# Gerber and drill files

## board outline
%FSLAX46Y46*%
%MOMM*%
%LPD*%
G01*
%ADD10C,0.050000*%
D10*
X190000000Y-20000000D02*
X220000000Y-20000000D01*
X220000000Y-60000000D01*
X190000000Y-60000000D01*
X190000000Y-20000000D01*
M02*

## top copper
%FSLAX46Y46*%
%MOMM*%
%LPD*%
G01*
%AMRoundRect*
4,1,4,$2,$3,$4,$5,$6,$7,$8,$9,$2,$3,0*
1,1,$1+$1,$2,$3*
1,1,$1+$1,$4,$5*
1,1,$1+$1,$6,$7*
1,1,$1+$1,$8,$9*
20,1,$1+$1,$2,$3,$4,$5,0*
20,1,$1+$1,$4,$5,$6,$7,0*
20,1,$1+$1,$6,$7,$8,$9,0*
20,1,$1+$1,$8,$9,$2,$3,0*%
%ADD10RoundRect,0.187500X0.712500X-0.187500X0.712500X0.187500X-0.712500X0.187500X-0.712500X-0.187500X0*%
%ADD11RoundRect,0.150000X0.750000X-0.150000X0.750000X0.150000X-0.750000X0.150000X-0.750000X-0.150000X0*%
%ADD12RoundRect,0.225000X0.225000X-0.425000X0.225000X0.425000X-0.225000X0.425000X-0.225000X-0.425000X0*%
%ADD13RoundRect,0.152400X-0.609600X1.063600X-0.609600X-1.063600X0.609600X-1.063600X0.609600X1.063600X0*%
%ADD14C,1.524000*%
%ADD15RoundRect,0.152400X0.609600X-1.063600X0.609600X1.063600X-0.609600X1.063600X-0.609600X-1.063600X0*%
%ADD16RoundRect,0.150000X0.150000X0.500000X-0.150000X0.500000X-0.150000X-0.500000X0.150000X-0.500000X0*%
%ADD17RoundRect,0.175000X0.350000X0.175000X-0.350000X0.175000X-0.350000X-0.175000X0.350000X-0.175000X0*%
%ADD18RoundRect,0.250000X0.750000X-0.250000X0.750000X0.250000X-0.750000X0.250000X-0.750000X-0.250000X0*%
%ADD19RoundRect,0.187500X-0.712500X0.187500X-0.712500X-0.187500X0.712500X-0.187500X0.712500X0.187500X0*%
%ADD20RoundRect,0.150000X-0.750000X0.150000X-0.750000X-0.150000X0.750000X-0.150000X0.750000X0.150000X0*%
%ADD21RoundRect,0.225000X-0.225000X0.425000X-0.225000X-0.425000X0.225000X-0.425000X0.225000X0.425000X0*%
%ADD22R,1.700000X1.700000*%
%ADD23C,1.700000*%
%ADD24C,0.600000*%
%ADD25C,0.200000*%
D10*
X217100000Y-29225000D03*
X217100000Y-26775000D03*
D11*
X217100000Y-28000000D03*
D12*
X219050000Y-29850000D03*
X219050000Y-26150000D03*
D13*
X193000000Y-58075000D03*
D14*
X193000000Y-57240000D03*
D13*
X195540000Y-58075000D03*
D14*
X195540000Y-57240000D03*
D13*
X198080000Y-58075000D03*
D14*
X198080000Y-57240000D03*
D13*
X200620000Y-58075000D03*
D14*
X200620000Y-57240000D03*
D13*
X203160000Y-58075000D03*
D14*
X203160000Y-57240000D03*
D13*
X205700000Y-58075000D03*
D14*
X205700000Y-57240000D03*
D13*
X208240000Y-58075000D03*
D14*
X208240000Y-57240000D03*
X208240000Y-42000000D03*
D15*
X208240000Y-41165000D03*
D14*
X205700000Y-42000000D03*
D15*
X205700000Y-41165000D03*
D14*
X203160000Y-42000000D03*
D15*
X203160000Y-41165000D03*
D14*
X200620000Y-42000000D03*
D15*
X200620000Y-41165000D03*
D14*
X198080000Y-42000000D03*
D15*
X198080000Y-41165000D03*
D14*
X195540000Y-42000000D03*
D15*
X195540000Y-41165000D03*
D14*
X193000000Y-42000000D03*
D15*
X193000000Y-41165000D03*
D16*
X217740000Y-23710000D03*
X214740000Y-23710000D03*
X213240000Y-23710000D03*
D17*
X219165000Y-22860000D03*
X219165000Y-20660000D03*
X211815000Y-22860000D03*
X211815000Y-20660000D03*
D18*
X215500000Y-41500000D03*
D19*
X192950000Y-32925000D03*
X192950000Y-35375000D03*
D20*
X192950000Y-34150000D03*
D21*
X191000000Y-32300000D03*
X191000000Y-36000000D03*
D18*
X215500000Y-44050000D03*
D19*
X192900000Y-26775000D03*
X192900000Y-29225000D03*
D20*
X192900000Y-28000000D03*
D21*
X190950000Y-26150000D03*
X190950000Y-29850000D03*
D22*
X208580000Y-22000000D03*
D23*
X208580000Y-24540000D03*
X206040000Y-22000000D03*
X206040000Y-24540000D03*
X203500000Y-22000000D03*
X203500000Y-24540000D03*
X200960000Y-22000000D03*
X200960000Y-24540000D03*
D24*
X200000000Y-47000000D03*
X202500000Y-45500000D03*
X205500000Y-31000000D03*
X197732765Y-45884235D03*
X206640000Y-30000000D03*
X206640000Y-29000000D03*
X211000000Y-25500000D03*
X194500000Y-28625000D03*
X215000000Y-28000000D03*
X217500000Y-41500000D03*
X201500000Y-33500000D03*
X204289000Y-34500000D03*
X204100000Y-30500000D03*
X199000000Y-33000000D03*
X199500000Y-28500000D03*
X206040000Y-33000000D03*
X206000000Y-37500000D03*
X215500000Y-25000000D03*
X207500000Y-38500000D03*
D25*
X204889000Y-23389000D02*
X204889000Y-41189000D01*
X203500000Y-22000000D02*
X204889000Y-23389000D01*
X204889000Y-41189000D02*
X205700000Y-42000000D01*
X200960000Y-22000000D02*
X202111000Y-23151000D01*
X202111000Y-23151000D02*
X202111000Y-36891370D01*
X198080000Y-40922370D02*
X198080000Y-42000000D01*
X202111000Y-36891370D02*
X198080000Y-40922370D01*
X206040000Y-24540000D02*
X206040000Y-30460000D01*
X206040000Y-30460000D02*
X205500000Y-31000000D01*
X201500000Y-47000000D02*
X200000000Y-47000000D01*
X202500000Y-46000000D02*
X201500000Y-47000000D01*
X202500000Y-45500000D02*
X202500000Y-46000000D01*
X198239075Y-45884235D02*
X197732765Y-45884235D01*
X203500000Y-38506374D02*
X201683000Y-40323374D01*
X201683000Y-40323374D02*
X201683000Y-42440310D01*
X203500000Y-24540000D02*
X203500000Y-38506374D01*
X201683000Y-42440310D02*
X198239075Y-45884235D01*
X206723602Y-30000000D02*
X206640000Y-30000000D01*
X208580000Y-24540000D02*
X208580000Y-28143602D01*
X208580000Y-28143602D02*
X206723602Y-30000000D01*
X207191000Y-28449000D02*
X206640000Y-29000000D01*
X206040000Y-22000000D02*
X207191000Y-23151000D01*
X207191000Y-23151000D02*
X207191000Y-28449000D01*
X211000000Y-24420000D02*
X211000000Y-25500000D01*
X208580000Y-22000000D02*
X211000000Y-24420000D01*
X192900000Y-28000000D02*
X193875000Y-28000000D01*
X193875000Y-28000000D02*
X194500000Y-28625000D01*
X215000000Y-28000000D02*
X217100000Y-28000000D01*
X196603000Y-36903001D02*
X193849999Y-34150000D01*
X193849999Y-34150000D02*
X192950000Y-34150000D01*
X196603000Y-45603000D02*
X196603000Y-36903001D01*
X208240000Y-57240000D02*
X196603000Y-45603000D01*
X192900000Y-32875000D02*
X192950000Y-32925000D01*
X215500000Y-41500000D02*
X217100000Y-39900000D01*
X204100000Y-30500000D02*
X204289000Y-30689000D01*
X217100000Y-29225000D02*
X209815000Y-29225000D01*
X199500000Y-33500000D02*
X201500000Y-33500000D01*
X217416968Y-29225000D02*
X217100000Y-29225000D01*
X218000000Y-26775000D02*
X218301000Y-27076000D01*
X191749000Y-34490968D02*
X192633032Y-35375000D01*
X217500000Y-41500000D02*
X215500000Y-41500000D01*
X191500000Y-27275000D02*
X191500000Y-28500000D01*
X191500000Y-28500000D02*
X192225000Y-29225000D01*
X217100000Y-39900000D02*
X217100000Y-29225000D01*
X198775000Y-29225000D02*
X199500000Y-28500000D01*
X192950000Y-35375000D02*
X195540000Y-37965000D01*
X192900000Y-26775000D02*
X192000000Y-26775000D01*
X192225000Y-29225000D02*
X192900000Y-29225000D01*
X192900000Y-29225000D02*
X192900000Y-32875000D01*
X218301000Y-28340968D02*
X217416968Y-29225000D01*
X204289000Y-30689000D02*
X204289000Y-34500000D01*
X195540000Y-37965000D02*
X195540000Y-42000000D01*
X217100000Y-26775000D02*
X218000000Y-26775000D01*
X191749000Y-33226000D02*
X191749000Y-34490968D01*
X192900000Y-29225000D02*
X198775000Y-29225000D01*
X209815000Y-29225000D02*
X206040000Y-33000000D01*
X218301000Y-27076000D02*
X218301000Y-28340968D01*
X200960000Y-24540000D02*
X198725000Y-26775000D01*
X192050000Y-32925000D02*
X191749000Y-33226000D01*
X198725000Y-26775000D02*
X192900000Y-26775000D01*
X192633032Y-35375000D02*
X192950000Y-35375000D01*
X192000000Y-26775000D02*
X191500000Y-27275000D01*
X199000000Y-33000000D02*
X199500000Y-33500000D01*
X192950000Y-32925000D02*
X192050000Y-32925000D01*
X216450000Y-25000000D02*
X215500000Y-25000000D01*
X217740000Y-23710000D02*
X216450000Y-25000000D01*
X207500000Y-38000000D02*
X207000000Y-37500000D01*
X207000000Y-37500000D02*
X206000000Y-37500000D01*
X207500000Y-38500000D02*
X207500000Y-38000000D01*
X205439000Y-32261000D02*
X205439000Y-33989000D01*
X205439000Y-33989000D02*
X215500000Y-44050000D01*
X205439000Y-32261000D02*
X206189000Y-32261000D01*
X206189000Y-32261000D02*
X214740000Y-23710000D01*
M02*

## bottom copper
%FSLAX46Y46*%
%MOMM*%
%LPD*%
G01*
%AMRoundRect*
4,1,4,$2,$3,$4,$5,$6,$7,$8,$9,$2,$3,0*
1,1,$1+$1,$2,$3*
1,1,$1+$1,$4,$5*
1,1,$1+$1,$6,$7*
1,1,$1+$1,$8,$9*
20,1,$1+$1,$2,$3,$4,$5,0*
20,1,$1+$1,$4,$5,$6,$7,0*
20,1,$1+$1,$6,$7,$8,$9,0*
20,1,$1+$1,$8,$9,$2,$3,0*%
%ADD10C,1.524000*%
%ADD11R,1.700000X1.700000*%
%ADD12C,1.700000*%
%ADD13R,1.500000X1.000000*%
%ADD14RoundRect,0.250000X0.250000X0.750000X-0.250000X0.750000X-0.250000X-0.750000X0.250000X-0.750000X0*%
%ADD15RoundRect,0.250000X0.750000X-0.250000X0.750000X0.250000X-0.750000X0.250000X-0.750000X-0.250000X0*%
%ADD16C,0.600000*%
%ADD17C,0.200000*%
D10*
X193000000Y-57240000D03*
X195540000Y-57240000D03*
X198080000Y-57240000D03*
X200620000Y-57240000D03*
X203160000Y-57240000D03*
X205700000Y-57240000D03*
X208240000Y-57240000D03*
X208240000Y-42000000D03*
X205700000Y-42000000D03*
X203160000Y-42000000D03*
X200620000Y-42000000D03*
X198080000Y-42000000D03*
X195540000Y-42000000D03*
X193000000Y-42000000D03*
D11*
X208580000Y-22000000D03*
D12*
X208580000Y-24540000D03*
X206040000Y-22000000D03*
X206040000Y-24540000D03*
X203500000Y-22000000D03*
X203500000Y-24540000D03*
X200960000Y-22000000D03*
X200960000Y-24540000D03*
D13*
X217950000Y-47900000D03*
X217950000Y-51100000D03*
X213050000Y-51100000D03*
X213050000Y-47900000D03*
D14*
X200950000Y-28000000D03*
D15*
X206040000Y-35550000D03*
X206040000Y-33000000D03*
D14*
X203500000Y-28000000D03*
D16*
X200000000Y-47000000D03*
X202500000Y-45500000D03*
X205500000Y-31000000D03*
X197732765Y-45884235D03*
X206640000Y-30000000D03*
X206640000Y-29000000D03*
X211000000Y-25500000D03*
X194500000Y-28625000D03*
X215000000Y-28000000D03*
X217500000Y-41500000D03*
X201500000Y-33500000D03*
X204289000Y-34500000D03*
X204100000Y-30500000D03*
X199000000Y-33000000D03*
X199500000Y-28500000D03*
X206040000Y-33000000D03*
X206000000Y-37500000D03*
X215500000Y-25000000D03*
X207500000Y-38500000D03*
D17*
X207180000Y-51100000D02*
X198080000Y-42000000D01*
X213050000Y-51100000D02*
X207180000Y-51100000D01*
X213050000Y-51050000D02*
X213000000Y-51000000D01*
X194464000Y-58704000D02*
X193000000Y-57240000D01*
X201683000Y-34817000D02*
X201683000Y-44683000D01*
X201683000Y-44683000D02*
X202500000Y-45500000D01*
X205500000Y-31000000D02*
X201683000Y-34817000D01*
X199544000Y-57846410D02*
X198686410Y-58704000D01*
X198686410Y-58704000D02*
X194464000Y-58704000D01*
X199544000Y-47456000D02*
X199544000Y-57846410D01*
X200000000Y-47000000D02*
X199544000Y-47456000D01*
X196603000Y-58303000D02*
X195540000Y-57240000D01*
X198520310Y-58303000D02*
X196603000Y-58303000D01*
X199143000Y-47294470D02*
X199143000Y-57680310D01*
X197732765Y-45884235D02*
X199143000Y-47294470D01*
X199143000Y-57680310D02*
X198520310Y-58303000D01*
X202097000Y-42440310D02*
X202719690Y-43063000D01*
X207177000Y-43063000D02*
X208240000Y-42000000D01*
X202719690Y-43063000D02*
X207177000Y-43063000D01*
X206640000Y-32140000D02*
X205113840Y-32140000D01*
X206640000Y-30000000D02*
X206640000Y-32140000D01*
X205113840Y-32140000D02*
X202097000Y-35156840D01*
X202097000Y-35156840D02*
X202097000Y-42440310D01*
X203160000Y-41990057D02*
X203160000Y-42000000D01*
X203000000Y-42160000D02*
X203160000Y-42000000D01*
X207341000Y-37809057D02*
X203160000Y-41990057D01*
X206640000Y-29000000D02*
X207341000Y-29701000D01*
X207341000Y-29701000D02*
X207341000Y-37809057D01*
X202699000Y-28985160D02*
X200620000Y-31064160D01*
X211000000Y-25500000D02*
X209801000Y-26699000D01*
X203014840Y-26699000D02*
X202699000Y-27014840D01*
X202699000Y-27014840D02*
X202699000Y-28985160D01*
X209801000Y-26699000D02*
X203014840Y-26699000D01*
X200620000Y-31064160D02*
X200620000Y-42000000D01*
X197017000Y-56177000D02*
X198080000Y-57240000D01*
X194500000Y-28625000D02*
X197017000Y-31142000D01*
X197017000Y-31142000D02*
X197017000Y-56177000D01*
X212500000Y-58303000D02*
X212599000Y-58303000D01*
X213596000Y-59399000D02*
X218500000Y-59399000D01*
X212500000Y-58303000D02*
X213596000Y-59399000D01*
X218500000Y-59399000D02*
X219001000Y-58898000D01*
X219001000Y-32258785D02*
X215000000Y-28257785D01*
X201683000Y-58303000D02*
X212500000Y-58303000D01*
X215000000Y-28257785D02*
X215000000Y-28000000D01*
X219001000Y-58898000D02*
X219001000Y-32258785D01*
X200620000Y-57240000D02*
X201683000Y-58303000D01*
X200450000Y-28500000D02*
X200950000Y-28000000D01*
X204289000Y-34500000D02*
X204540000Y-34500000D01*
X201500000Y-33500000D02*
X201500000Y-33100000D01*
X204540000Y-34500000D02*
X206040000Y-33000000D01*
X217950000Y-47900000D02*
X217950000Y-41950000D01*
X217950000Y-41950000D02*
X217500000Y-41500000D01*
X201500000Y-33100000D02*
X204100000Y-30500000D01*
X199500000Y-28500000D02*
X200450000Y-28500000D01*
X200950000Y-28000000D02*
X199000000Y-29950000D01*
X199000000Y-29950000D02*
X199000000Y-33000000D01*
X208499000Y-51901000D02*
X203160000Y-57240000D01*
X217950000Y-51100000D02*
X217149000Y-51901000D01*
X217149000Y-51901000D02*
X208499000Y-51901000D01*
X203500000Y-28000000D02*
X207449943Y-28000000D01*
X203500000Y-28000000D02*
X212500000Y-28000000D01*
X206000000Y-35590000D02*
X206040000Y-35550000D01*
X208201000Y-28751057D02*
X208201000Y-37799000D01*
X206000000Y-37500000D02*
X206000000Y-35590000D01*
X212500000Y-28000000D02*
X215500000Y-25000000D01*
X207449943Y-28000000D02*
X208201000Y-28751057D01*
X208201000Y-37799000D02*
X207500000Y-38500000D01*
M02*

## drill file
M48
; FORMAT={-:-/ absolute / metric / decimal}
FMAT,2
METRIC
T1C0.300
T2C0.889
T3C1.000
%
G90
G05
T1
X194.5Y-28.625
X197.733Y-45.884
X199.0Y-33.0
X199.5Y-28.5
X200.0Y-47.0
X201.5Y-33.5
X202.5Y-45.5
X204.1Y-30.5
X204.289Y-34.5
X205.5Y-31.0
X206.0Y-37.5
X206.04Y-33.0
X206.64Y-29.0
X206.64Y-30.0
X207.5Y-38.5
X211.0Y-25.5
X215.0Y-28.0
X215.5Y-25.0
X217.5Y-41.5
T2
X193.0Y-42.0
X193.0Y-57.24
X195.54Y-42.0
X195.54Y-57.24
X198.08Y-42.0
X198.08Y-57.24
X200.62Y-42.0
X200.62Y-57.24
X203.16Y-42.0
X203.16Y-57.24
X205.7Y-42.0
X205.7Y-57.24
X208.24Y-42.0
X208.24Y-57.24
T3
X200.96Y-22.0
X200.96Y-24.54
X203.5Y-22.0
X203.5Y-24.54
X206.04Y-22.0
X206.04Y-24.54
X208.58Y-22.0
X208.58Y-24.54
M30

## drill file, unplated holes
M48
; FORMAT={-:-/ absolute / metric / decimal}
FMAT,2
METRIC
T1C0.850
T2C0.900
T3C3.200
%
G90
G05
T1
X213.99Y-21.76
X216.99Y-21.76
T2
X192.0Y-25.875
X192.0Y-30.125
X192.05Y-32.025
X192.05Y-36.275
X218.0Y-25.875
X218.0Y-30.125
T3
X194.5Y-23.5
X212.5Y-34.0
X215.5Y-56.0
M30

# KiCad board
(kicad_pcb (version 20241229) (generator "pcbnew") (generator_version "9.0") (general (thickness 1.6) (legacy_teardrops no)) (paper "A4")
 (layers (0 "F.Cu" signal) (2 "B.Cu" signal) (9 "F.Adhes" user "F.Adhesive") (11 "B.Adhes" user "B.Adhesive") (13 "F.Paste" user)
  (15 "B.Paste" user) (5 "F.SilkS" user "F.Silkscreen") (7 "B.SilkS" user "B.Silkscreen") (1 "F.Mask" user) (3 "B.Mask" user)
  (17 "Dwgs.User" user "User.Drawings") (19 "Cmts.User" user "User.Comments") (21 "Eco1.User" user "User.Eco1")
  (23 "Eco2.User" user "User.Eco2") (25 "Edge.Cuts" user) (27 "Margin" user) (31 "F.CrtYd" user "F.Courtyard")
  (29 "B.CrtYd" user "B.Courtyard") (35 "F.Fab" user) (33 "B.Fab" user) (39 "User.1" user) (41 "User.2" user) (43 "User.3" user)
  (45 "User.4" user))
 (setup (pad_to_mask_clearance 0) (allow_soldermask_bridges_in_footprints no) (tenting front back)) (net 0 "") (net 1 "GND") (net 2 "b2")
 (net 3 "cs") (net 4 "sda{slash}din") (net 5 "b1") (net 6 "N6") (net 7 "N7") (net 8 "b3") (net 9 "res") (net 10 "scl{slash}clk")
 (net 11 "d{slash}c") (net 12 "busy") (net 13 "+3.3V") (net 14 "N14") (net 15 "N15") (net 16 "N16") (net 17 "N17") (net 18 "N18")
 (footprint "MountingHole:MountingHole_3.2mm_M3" (layer "F.Cu") (at 215.5 56)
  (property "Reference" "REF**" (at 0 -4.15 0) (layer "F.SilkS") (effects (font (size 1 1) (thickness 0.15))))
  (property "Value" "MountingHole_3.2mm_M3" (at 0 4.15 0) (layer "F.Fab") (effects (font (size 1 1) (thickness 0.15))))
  (pad "" np_thru_hole circle (at 0 0) (size 3.2 3.2) (drill 3.2) (layers "*.Cu" "*.Mask")))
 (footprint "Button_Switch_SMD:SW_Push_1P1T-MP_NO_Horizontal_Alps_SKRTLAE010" (layer "F.Cu") (at 218 28 90)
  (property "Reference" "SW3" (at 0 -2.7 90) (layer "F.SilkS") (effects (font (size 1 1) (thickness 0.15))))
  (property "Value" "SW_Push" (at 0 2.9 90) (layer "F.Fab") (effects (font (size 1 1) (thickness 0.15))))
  (pad "" np_thru_hole circle (at -2.125 0 90) (size 0.9 0.9) (drill 0.9) (layers "*.Cu" "*.Mask"))
  (pad "" np_thru_hole circle (at 2.125 0 90) (size 0.9 0.9) (drill 0.9) (layers "*.Cu" "*.Mask"))
  (pad "1" smd roundrect (at -1.225 -0.9 90) (size 0.75 1.8) (layers "F.Cu" "F.Mask" "F.Paste") (roundrect_rratio 0.25) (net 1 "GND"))
  (pad "1" smd roundrect (at 1.225 -0.9 90) (size 0.75 1.8) (layers "F.Cu" "F.Mask" "F.Paste") (roundrect_rratio 0.25) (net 1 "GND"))
  (pad "2" smd roundrect (at 0 -0.9 90) (size 0.6 1.8) (layers "F.Cu" "F.Mask" "F.Paste") (roundrect_rratio 0.25) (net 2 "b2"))
  (pad "MP" smd roundrect (at -1.85 1.05 90) (size 1.3 0.9) (layers "F.Cu" "F.Mask" "F.Paste") (roundrect_rratio 0.25))
  (pad "MP" smd roundrect (at 1.85 1.05 90) (size 1.3 0.9) (layers "F.Cu" "F.Mask" "F.Paste") (roundrect_rratio 0.25)))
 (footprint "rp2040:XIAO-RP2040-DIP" (layer "F.Cu") (at 200.62 49.62 90)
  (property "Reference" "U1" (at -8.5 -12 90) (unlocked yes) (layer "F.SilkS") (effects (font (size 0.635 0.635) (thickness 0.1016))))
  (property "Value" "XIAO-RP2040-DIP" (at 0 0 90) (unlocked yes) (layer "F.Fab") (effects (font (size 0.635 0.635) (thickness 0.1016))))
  (pad "1" smd roundrect (at -8.455 -7.62 270) (size 2.432 1.524) (layers "F.Cu" "F.Mask") (roundrect_rratio 0.1) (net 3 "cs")
   (thermal_bridge_angle 45))
  (pad "1" thru_hole circle (at -7.62 -7.62 270) (size 1.524 1.524) (drill 0.889) (layers "*.Cu" "*.Mask") (remove_unused_layers no)
   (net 3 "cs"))
  (pad "2" smd roundrect (at -8.455 -5.08 270) (size 2.432 1.524) (layers "F.Cu" "F.Mask") (roundrect_rratio 0.1) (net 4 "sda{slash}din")
   (thermal_bridge_angle 45))
  (pad "2" thru_hole circle (at -7.62 -5.08 270) (size 1.524 1.524) (drill 0.889) (layers "*.Cu" "*.Mask") (remove_unused_layers no)
   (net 4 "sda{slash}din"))
  (pad "3" smd roundrect (at -8.455 -2.54 270) (size 2.432 1.524) (layers "F.Cu" "F.Mask") (roundrect_rratio 0.1) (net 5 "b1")
   (thermal_bridge_angle 45))
  (pad "3" thru_hole circle (at -7.62 -2.54 270) (size 1.524 1.524) (drill 0.889) (layers "*.Cu" "*.Mask") (remove_unused_layers no)
   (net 5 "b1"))
  (pad "4" smd roundrect (at -8.455 0 270) (size 2.432 1.524) (layers "F.Cu" "F.Mask") (roundrect_rratio 0.1) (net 2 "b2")
   (thermal_bridge_angle 45))
  (pad "4" thru_hole circle (at -7.62 0 270) (size 1.524 1.524) (drill 0.889) (layers "*.Cu" "*.Mask") (remove_unused_layers no)
   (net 2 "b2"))
  (pad "5" smd roundrect (at -8.455 2.54 270) (size 2.432 1.524) (layers "F.Cu" "F.Mask") (roundrect_rratio 0.1) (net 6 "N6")
   (thermal_bridge_angle 45))
  (pad "5" thru_hole circle (at -7.62 2.54 270) (size 1.524 1.524) (drill 0.889) (layers "*.Cu" "*.Mask") (remove_unused_layers no)
   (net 6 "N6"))
  (pad "6" smd roundrect (at -8.455 5.08 270) (size 2.432 1.524) (layers "F.Cu" "F.Mask") (roundrect_rratio 0.1) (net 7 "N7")
   (thermal_bridge_angle 45))
  (pad "6" thru_hole circle (at -7.62 5.08 270) (size 1.524 1.524) (drill 0.889) (layers "*.Cu" "*.Mask") (remove_unused_layers no)
   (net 7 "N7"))
  (pad "7" smd roundrect (at -8.455 7.62 270) (size 2.432 1.524) (layers "F.Cu" "F.Mask") (roundrect_rratio 0.1) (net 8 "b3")
   (thermal_bridge_angle 45))
  (pad "7" thru_hole circle (at -7.62 7.62 270) (size 1.524 1.524) (drill 0.889) (layers "*.Cu" "*.Mask") (remove_unused_layers no)
   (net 8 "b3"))
  (pad "8" thru_hole circle (at 7.62 7.62 90) (size 1.524 1.524) (drill 0.889) (layers "*.Cu" "*.Mask") (remove_unused_layers no)
   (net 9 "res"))
  (pad "8" smd roundrect (at 8.455 7.62 90) (size 2.432 1.524) (layers "F.Cu" "F.Mask") (roundrect_rratio 0.1) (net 9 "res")
   (thermal_bridge_angle 45))
  (pad "9" thru_hole circle (at 7.62 5.08 90) (size 1.524 1.524) (drill 0.889) (layers "*.Cu" "*.Mask") (remove_unused_layers no)
   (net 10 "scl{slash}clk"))
  (pad "9" smd roundrect (at 8.455 5.08 90) (size 2.432 1.524) (layers "F.Cu" "F.Mask") (roundrect_rratio 0.1) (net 10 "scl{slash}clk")
   (thermal_bridge_angle 45))
  (pad "10" thru_hole circle (at 7.62 2.54 90) (size 1.524 1.524) (drill 0.889) (layers "*.Cu" "*.Mask") (remove_unused_layers no)
   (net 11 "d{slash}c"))
  (pad "10" smd roundrect (at 8.455 2.54 90) (size 2.432 1.524) (layers "F.Cu" "F.Mask") (roundrect_rratio 0.1) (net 11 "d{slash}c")
   (thermal_bridge_angle 45))
  (pad "11" thru_hole circle (at 7.62 0 90) (size 1.524 1.524) (drill 0.889) (layers "*.Cu" "*.Mask") (remove_unused_layers no)
   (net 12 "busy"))
  (pad "11" smd roundrect (at 8.455 0 90) (size 2.432 1.524) (layers "F.Cu" "F.Mask") (roundrect_rratio 0.1) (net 12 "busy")
   (thermal_bridge_angle 45))
  (pad "12" thru_hole circle (at 7.62 -2.54 90) (size 1.524 1.524) (drill 0.889) (layers "*.Cu" "*.Mask") (remove_unused_layers no)
   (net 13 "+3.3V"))
  (pad "12" smd roundrect (at 8.455 -2.54 90) (size 2.432 1.524) (layers "F.Cu" "F.Mask") (roundrect_rratio 0.1) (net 13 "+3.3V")
   (thermal_bridge_angle 45))
  (pad "13" thru_hole circle (at 7.62 -5.08 90) (size 1.524 1.524) (drill 0.889) (layers "*.Cu" "*.Mask") (remove_unused_layers no)
   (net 1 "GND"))
  (pad "13" smd roundrect (at 8.455 -5.08 90) (size 2.432 1.524) (layers "F.Cu" "F.Mask") (roundrect_rratio 0.1) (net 1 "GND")
   (thermal_bridge_angle 45))
  (pad "14" thru_hole circle (at 7.62 -7.62 90) (size 1.524 1.524) (drill 0.889) (layers "*.Cu" "*.Mask") (remove_unused_layers no)
   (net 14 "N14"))
  (pad "14" smd roundrect (at 8.455 -7.62 90) (size 2.432 1.524) (layers "F.Cu" "F.Mask") (roundrect_rratio 0.1) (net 14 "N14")
   (thermal_bridge_angle 45)))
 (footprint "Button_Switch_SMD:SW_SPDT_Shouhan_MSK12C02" (layer "F.Cu") (at 215.49 21.76 180)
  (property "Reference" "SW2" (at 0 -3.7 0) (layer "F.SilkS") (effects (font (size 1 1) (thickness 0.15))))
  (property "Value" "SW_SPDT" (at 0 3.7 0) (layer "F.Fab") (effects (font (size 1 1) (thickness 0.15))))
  (pad "" np_thru_hole circle (at -1.5 0 180) (size 0.85 0.85) (drill 0.85) (layers "*.Mask"))
  (pad "" np_thru_hole circle (at 1.5 0 180) (size 0.85 0.85) (drill 0.85) (layers "*.Mask"))
  (pad "1" smd roundrect (at -2.25 -1.95 180) (size 0.6 1.3) (layers "F.Cu" "F.Mask" "F.Paste") (roundrect_rratio 0.25) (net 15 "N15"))
  (pad "2" smd roundrect (at 0.75 -1.95 180) (size 0.6 1.3) (layers "F.Cu" "F.Mask" "F.Paste") (roundrect_rratio 0.25) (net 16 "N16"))
  (pad "3" smd roundrect (at 2.25 -1.95 180) (size 0.6 1.3) (layers "F.Cu" "F.Mask" "F.Paste") (roundrect_rratio 0.25) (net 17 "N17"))
  (pad "SH" smd roundrect (at -3.675 -1.1 180) (size 1.05 0.7) (layers "F.Cu" "F.Mask" "F.Paste") (roundrect_rratio 0.25))
  (pad "SH" smd roundrect (at -3.675 1.1 180) (size 1.05 0.7) (layers "F.Cu" "F.Mask" "F.Paste") (roundrect_rratio 0.25))
  (pad "SH" smd roundrect (at 3.675 -1.1 180) (size 1.05 0.7) (layers "F.Cu" "F.Mask" "F.Paste") (roundrect_rratio 0.25))
  (pad "SH" smd roundrect (at 3.675 1.1 180) (size 1.05 0.7) (layers "F.Cu" "F.Mask" "F.Paste") (roundrect_rratio 0.25)))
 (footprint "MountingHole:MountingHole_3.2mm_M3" (layer "F.Cu") (at 212.5 34)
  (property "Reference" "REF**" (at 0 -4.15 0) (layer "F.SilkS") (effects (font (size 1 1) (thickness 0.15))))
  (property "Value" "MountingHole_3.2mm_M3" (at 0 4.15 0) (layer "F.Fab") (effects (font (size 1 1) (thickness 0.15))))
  (pad "" np_thru_hole circle (at 0 0) (size 3.2 3.2) (drill 3.2) (layers "*.Cu" "*.Mask")))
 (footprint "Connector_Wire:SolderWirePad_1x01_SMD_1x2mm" (layer "F.Cu") (at 215.5 41.5 90)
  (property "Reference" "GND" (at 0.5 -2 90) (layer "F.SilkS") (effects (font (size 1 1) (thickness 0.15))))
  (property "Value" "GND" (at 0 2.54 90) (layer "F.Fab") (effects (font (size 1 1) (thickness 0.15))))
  (pad "1" smd roundrect (at 0 0 90) (size 1 2) (layers "F.Cu" "F.Mask") (roundrect_rratio 0.25) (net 1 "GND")))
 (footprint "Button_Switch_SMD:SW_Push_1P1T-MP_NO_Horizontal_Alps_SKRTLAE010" (layer "F.Cu") (at 192.05 34.15 -90)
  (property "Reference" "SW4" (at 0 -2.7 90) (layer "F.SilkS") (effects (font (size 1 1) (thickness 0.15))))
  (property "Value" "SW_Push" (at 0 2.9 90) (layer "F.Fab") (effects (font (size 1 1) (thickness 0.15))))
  (pad "" np_thru_hole circle (at -2.125 0 270) (size 0.9 0.9) (drill 0.9) (layers "*.Cu" "*.Mask"))
  (pad "" np_thru_hole circle (at 2.125 0 270) (size 0.9 0.9) (drill 0.9) (layers "*.Cu" "*.Mask"))
  (pad "1" smd roundrect (at -1.225 -0.9 270) (size 0.75 1.8) (layers "F.Cu" "F.Mask" "F.Paste") (roundrect_rratio 0.25) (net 1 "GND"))
  (pad "1" smd roundrect (at 1.225 -0.9 270) (size 0.75 1.8) (layers "F.Cu" "F.Mask" "F.Paste") (roundrect_rratio 0.25) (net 1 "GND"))
  (pad "2" smd roundrect (at 0 -0.9 270) (size 0.6 1.8) (layers "F.Cu" "F.Mask" "F.Paste") (roundrect_rratio 0.25) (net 8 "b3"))
  (pad "MP" smd roundrect (at -1.85 1.05 270) (size 1.3 0.9) (layers "F.Cu" "F.Mask" "F.Paste") (roundrect_rratio 0.25))
  (pad "MP" smd roundrect (at 1.85 1.05 270) (size 1.3 0.9) (layers "F.Cu" "F.Mask" "F.Paste") (roundrect_rratio 0.25)))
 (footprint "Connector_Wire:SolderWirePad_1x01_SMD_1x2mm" (layer "F.Cu") (at 215.5 44.05 90)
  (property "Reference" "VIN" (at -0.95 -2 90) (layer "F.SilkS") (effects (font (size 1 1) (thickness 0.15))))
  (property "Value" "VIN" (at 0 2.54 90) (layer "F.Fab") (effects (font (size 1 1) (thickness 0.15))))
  (pad "1" smd roundrect (at 0 0 90) (size 1 2) (layers "F.Cu" "F.Mask") (roundrect_rratio 0.25) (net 16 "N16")))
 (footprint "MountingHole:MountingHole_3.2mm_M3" (layer "F.Cu") (at 194.5 23.5)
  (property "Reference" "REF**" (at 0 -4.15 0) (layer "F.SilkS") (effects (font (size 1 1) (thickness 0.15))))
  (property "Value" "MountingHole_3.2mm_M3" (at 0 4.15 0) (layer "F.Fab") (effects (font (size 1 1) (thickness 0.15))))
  (pad "" np_thru_hole circle (at 0 0) (size 3.2 3.2) (drill 3.2) (layers "*.Cu" "*.Mask")))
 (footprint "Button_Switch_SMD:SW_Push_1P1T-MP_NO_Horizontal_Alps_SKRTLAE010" (layer "F.Cu") (at 192 28 -90)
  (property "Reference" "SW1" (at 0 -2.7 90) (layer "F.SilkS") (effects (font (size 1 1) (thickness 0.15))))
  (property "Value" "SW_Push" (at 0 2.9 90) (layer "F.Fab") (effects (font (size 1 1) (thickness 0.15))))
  (pad "" np_thru_hole circle (at -2.125 0 270) (size 0.9 0.9) (drill 0.9) (layers "*.Cu" "*.Mask"))
  (pad "" np_thru_hole circle (at 2.125 0 270) (size 0.9 0.9) (drill 0.9) (layers "*.Cu" "*.Mask"))
  (pad "1" smd roundrect (at -1.225 -0.9 270) (size 0.75 1.8) (layers "F.Cu" "F.Mask" "F.Paste") (roundrect_rratio 0.25) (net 1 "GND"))
  (pad "1" smd roundrect (at 1.225 -0.9 270) (size 0.75 1.8) (layers "F.Cu" "F.Mask" "F.Paste") (roundrect_rratio 0.25) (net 1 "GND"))
  (pad "2" smd roundrect (at 0 -0.9 270) (size 0.6 1.8) (layers "F.Cu" "F.Mask" "F.Paste") (roundrect_rratio 0.25) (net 5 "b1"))
  (pad "MP" smd roundrect (at -1.85 1.05 270) (size 1.3 0.9) (layers "F.Cu" "F.Mask" "F.Paste") (roundrect_rratio 0.25))
  (pad "MP" smd roundrect (at 1.85 1.05 270) (size 1.3 0.9) (layers "F.Cu" "F.Mask" "F.Paste") (roundrect_rratio 0.25)))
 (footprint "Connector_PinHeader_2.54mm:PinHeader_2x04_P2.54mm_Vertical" (layer "F.Cu") (at 208.58 22 -90)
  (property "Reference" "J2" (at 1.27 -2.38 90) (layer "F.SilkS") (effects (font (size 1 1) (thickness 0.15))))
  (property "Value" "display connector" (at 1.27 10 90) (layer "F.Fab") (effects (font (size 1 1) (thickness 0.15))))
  (pad "1" thru_hole rect (at 0 0 270) (size 1.7 1.7) (drill 1) (layers "*.Cu" "*.Mask") (remove_unused_layers no) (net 12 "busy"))
  (pad "2" thru_hole circle (at 2.54 0 270) (size 1.7 1.7) (drill 1) (layers "*.Cu" "*.Mask") (remove_unused_layers no) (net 9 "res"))
  (pad "3" thru_hole circle (at 0 2.54 270) (size 1.7 1.7) (drill 1) (layers "*.Cu" "*.Mask") (remove_unused_layers no) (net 11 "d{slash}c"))
  (pad "4" thru_hole circle (at 2.54 2.54 270) (size 1.7 1.7) (drill 1) (layers "*.Cu" "*.Mask") (remove_unused_layers no) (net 3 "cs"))
  (pad "5" thru_hole circle (at 0 5.08 270) (size 1.7 1.7) (drill 1) (layers "*.Cu" "*.Mask") (remove_unused_layers no)
   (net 10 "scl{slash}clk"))
  (pad "6" thru_hole circle (at 2.54 5.08 270) (size 1.7 1.7) (drill 1) (layers "*.Cu" "*.Mask") (remove_unused_layers no)
   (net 4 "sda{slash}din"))
  (pad "7" thru_hole circle (at 0 7.62 270) (size 1.7 1.7) (drill 1) (layers "*.Cu" "*.Mask") (remove_unused_layers no) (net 13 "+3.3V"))
  (pad "8" thru_hole circle (at 2.54 7.62 270) (size 1.7 1.7) (drill 1) (layers "*.Cu" "*.Mask") (remove_unused_layers no) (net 1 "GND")))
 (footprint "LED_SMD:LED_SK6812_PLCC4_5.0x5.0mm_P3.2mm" (layer "B.Cu") (at 215.5 49.5 180)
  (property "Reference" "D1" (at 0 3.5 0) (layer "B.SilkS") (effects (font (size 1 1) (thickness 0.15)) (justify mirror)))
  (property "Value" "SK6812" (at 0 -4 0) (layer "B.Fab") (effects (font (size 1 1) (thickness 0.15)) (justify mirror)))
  (pad "1" smd rect (at -2.45 1.6) (size 1.5 1) (layers "B.Cu" "B.Mask" "B.Paste") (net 1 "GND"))
  (pad "2" smd rect (at -2.45 -1.6) (size 1.5 1) (layers "B.Cu" "B.Mask" "B.Paste") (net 6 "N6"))
  (pad "3" smd rect (at 2.45 -1.6) (size 1.5 1) (layers "B.Cu" "B.Mask" "B.Paste") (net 13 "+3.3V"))
  (pad "4" smd rect (at 2.45 1.6) (size 1.5 1) (layers "B.Cu" "B.Mask" "B.Paste") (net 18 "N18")))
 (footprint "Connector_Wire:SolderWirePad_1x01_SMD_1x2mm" (layer "B.Cu") (at 200.95 28 180)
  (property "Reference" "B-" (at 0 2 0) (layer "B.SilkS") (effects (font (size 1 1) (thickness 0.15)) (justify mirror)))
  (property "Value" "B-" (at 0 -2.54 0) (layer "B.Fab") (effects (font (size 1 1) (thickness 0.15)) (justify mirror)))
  (pad "1" smd roundrect (at 0 0 180) (size 1 2) (layers "B.Cu" "B.Mask") (roundrect_rratio 0.25) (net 1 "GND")))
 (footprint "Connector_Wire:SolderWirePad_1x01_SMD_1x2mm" (layer "B.Cu") (at 206.04 35.55 90)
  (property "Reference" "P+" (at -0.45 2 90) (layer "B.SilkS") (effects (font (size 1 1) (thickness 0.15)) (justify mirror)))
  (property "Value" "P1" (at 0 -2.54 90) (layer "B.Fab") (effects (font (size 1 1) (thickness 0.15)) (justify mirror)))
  (pad "1" smd roundrect (at 0 0 90) (size 1 2) (layers "B.Cu" "B.Mask") (roundrect_rratio 0.25) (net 15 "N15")))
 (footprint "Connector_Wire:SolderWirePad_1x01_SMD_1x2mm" (layer "B.Cu") (at 206.04 33 90)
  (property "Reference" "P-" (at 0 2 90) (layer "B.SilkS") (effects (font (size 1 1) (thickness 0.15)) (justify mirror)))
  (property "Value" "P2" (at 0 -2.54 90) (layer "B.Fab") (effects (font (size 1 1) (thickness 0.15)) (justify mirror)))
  (pad "1" smd roundrect (at 0 0 90) (size 1 2) (layers "B.Cu" "B.Mask") (roundrect_rratio 0.25) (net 1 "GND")))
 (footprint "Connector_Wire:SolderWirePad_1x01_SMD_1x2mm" (layer "B.Cu") (at 203.5 28 180)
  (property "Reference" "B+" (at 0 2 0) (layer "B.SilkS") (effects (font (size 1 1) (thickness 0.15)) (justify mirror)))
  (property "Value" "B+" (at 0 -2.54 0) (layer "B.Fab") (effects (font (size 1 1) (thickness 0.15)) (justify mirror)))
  (pad "1" smd roundrect (at 0 0 180) (size 1 2) (layers "B.Cu" "B.Mask") (roundrect_rratio 0.25) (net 15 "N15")))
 (gr_rect (start 190 20) (end 220 60) (stroke (width 0.05) (type default)) (fill no) (layer "Edge.Cuts"))
 (segment (start 204.889 23.389) (end 204.889 41.189) (width 0.2) (layer "F.Cu") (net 10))
 (segment (start 203.5 22) (end 204.889 23.389) (width 0.2) (layer "F.Cu") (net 10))
 (segment (start 204.889 41.189) (end 205.7 42) (width 0.2) (layer "F.Cu") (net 10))
 (segment (start 200.96 22) (end 202.111 23.151) (width 0.2) (layer "F.Cu") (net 13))
 (segment (start 202.111 23.151) (end 202.111 36.89137) (width 0.2) (layer "F.Cu") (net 13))
 (segment (start 198.08 40.92237) (end 198.08 42) (width 0.2) (layer "F.Cu") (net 13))
 (segment (start 202.111 36.89137) (end 198.08 40.92237) (width 0.2) (layer "F.Cu") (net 13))
 (segment (start 207.18 51.1) (end 198.08 42) (width 0.2) (layer "B.Cu") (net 13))
 (segment (start 213.05 51.1) (end 207.18 51.1) (width 0.2) (layer "B.Cu") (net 13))
 (segment (start 213.05 51.05) (end 213 51) (width 0.2) (layer "B.Cu") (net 13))
 (segment (start 206.04 24.54) (end 206.04 30.46) (width 0.2) (layer "F.Cu") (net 3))
 (segment (start 206.04 30.46) (end 205.5 31) (width 0.2) (layer "F.Cu") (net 3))
 (segment (start 201.5 47) (end 200 47) (width 0.2) (layer "F.Cu") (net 3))
 (segment (start 202.5 46) (end 201.5 47) (width 0.2) (layer "F.Cu") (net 3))
 (segment (start 202.5 45.5) (end 202.5 46) (width 0.2) (layer "F.Cu") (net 3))
 (via (at 200 47) (size 0.6) (drill 0.3) (layers "F.Cu" "B.Cu") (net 3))
 (via (at 202.5 45.5) (size 0.6) (drill 0.3) (layers "F.Cu" "B.Cu") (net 3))
 (via (at 205.5 31) (size 0.6) (drill 0.3) (layers "F.Cu" "B.Cu") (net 3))
 (segment (start 194.464 58.704) (end 193 57.24) (width 0.2) (layer "B.Cu") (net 3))
 (segment (start 201.683 34.817) (end 201.683 44.683) (width 0.2) (layer "B.Cu") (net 3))
 (segment (start 201.683 44.683) (end 202.5 45.5) (width 0.2) (layer "B.Cu") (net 3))
 (segment (start 205.5 31) (end 201.683 34.817) (width 0.2) (layer "B.Cu") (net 3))
 (segment (start 199.544 57.84641) (end 198.68641 58.704) (width 0.2) (layer "B.Cu") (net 3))
 (segment (start 198.68641 58.704) (end 194.464 58.704) (width 0.2) (layer "B.Cu") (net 3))
 (segment (start 199.544 47.456) (end 199.544 57.84641) (width 0.2) (layer "B.Cu") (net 3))
 (segment (start 200 47) (end 199.544 47.456) (width 0.2) (layer "B.Cu") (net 3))
 (segment (start 198.239075 45.884235) (end 197.732765 45.884235) (width 0.2) (layer "F.Cu") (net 4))
 (segment (start 203.5 38.506374) (end 201.683 40.323374) (width 0.2) (layer "F.Cu") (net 4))
 (segment (start 201.683 40.323374) (end 201.683 42.44031) (width 0.2) (layer "F.Cu") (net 4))
 (segment (start 203.5 24.54) (end 203.5 38.506374) (width 0.2) (layer "F.Cu") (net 4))
 (segment (start 201.683 42.44031) (end 198.239075 45.884235) (width 0.2) (layer "F.Cu") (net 4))
 (via (at 197.732765 45.884235) (size 0.6) (drill 0.3) (layers "F.Cu" "B.Cu") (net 4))
 (segment (start 196.603 58.303) (end 195.54 57.24) (width 0.2) (layer "B.Cu") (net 4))
 (segment (start 198.52031 58.303) (end 196.603 58.303) (width 0.2) (layer "B.Cu") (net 4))
 (segment (start 199.143 47.29447) (end 199.143 57.68031) (width 0.2) (layer "B.Cu") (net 4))
 (segment (start 197.732765 45.884235) (end 199.143 47.29447) (width 0.2) (layer "B.Cu") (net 4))
 (segment (start 199.143 57.68031) (end 198.52031 58.303) (width 0.2) (layer "B.Cu") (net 4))
 (segment (start 206.723602 30) (end 206.64 30) (width 0.2) (layer "F.Cu") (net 9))
 (segment (start 208.58 24.54) (end 208.58 28.143602) (width 0.2) (layer "F.Cu") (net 9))
 (segment (start 208.58 28.143602) (end 206.723602 30) (width 0.2) (layer "F.Cu") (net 9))
 (via (at 206.64 30) (size 0.6) (drill 0.3) (layers "F.Cu" "B.Cu") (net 9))
 (segment (start 202.097 42.44031) (end 202.71969 43.063) (width 0.2) (layer "B.Cu") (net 9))
 (segment (start 207.177 43.063) (end 208.24 42) (width 0.2) (layer "B.Cu") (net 9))
 (segment (start 202.71969 43.063) (end 207.177 43.063) (width 0.2) (layer "B.Cu") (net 9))
 (segment (start 206.64 32.14) (end 205.11384 32.14) (width 0.2) (layer "B.Cu") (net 9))
 (segment (start 206.64 30) (end 206.64 32.14) (width 0.2) (layer "B.Cu") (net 9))
 (segment (start 205.11384 32.14) (end 202.097 35.15684) (width 0.2) (layer "B.Cu") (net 9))
 (segment (start 202.097 35.15684) (end 202.097 42.44031) (width 0.2) (layer "B.Cu") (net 9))
 (segment (start 207.191 28.449) (end 206.64 29) (width 0.2) (layer "F.Cu") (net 11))
 (segment (start 206.04 22) (end 207.191 23.151) (width 0.2) (layer "F.Cu") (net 11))
 (segment (start 207.191 23.151) (end 207.191 28.449) (width 0.2) (layer "F.Cu") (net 11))
 (via (at 206.64 29) (size 0.6) (drill 0.3) (layers "F.Cu" "B.Cu") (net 11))
 (segment (start 203.16 41.990057) (end 203.16 42) (width 0.2) (layer "B.Cu") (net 11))
 (segment (start 203 42.16) (end 203.16 42) (width 0.2) (layer "B.Cu") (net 11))
 (segment (start 207.341 37.809057) (end 203.16 41.990057) (width 0.2) (layer "B.Cu") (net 11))
 (segment (start 206.64 29) (end 207.341 29.701) (width 0.2) (layer "B.Cu") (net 11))
 (segment (start 207.341 29.701) (end 207.341 37.809057) (width 0.2) (layer "B.Cu") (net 11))
 (segment (start 211 24.42) (end 211 25.5) (width 0.2) (layer "F.Cu") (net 12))
 (segment (start 208.58 22) (end 211 24.42) (width 0.2) (layer "F.Cu") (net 12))
 (via (at 211 25.5) (size 0.6) (drill 0.3) (layers "F.Cu" "B.Cu") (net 12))
 (segment (start 202.699 28.98516) (end 200.62 31.06416) (width 0.2) (layer "B.Cu") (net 12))
 (segment (start 211 25.5) (end 209.801 26.699) (width 0.2) (layer "B.Cu") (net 12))
 (segment (start 203.01484 26.699) (end 202.699 27.01484) (width 0.2) (layer "B.Cu") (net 12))
 (segment (start 202.699 27.01484) (end 202.699 28.98516) (width 0.2) (layer "B.Cu") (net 12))
 (segment (start 209.801 26.699) (end 203.01484 26.699) (width 0.2) (layer "B.Cu") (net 12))
 (segment (start 200.62 31.06416) (end 200.62 42) (width 0.2) (layer "B.Cu") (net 12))
 (segment (start 192.9 28) (end 193.875 28) (width 0.2) (layer "F.Cu") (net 5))
 (segment (start 193.875 28) (end 194.5 28.625) (width 0.2) (layer "F.Cu") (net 5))
 (via (at 194.5 28.625) (size 0.6) (drill 0.3) (layers "F.Cu" "B.Cu") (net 5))
 (segment (start 197.017 56.177) (end 198.08 57.24) (width 0.2) (layer "B.Cu") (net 5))
 (segment (start 194.5 28.625) (end 197.017 31.142) (width 0.2) (layer "B.Cu") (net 5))
 (segment (start 197.017 31.142) (end 197.017 56.177) (width 0.2) (layer "B.Cu") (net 5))
 (segment (start 215 28) (end 217.1 28) (width 0.2) (layer "F.Cu") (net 2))
 (via (at 215 28) (size 0.6) (drill 0.3) (layers "F.Cu" "B.Cu") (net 2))
 (segment (start 212.5 58.303) (end 212.599 58.303) (width 0.2) (layer "B.Cu") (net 2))
 (segment (start 213.596 59.399) (end 218.5 59.399) (width 0.2) (layer "B.Cu") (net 2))
 (segment (start 212.5 58.303) (end 213.596 59.399) (width 0.2) (layer "B.Cu") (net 2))
 (segment (start 218.5 59.399) (end 219.001 58.898) (width 0.2) (layer "B.Cu") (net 2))
 (segment (start 219.001 32.258785) (end 215 28.257785) (width 0.2) (layer "B.Cu") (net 2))
 (segment (start 201.683 58.303) (end 212.5 58.303) (width 0.2) (layer "B.Cu") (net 2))
 (segment (start 215 28.257785) (end 215 28) (width 0.2) (layer "B.Cu") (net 2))
 (segment (start 219.001 58.898) (end 219.001 32.258785) (width 0.2) (layer "B.Cu") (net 2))
 (segment (start 200.62 57.24) (end 201.683 58.303) (width 0.2) (layer "B.Cu") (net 2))
 (segment (start 196.603 36.903001) (end 193.849999 34.15) (width 0.2) (layer "F.Cu") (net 8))
 (segment (start 193.849999 34.15) (end 192.95 34.15) (width 0.2) (layer "F.Cu") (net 8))
 (segment (start 196.603 45.603) (end 196.603 36.903001) (width 0.2) (layer "F.Cu") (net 8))
 (segment (start 208.24 57.24) (end 196.603 45.603) (width 0.2) (layer "F.Cu") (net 8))
 (segment (start 192.9 32.875) (end 192.95 32.925) (width 0.2) (layer "F.Cu") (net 1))
 (segment (start 215.5 41.5) (end 217.1 39.9) (width 0.2) (layer "F.Cu") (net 1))
 (segment (start 204.1 30.5) (end 204.289 30.689) (width 0.2) (layer "F.Cu") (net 1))
 (segment (start 217.1 29.225) (end 209.815 29.225) (width 0.2) (layer "F.Cu") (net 1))
 (segment (start 199.5 33.5) (end 201.5 33.5) (width 0.2) (layer "F.Cu") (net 1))
 (segment (start 217.416968 29.225) (end 217.1 29.225) (width 0.2) (layer "F.Cu") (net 1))
 (segment (start 218 26.775) (end 218.301 27.076) (width 0.2) (layer "F.Cu") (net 1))
 (segment (start 191.749 34.490968) (end 192.633032 35.375) (width 0.2) (layer "F.Cu") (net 1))
 (segment (start 217.5 41.5) (end 215.5 41.5) (width 0.2) (layer "F.Cu") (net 1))
 (segment (start 191.5 27.275) (end 191.5 28.5) (width 0.2) (layer "F.Cu") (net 1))
 (segment (start 191.5 28.5) (end 192.225 29.225) (width 0.2) (layer "F.Cu") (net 1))
 (segment (start 217.1 39.9) (end 217.1 29.225) (width 0.2) (layer "F.Cu") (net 1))
 (segment (start 198.775 29.225) (end 199.5 28.5) (width 0.2) (layer "F.Cu") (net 1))
 (segment (start 192.95 35.375) (end 195.54 37.965) (width 0.2) (layer "F.Cu") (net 1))
 (segment (start 192.9 26.775) (end 192 26.775) (width 0.2) (layer "F.Cu") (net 1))
 (segment (start 192.225 29.225) (end 192.9 29.225) (width 0.2) (layer "F.Cu") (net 1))
 (segment (start 192.9 29.225) (end 192.9 32.875) (width 0.2) (layer "F.Cu") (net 1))
 (segment (start 218.301 28.340968) (end 217.416968 29.225) (width 0.2) (layer "F.Cu") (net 1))
 (segment (start 204.289 30.689) (end 204.289 34.5) (width 0.2) (layer "F.Cu") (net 1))
 (segment (start 195.54 37.965) (end 195.54 42) (width 0.2) (layer "F.Cu") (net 1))
 (segment (start 217.1 26.775) (end 218 26.775) (width 0.2) (layer "F.Cu") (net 1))
 (segment (start 191.749 33.226) (end 191.749 34.490968) (width 0.2) (layer "F.Cu") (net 1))
 (segment (start 192.9 29.225) (end 198.775 29.225) (width 0.2) (layer "F.Cu") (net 1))
 (segment (start 209.815 29.225) (end 206.04 33) (width 0.2) (layer "F.Cu") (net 1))
 (segment (start 218.301 27.076) (end 218.301 28.340968) (width 0.2) (layer "F.Cu") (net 1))
 (segment (start 200.96 24.54) (end 198.725 26.775) (width 0.2) (layer "F.Cu") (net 1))
 (segment (start 192.05 32.925) (end 191.749 33.226) (width 0.2) (layer "F.Cu") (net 1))
 (segment (start 198.725 26.775) (end 192.9 26.775) (width 0.2) (layer "F.Cu") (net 1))
 (segment (start 192.633032 35.375) (end 192.95 35.375) (width 0.2) (layer "F.Cu") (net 1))
 (segment (start 192 26.775) (end 191.5 27.275) (width 0.2) (layer "F.Cu") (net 1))
 (segment (start 199 33) (end 199.5 33.5) (width 0.2) (layer "F.Cu") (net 1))
 (segment (start 192.95 32.925) (end 192.05 32.925) (width 0.2) (layer "F.Cu") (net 1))
 (via (at 217.5 41.5) (size 0.6) (drill 0.3) (layers "F.Cu" "B.Cu") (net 1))
 (via (at 201.5 33.5) (size 0.6) (drill 0.3) (layers "F.Cu" "B.Cu") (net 1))
 (via (at 204.289 34.5) (size 0.6) (drill 0.3) (layers "F.Cu" "B.Cu") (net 1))
 (via (at 204.1 30.5) (size 0.6) (drill 0.3) (layers "F.Cu" "B.Cu") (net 1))
 (via (at 199 33) (size 0.6) (drill 0.3) (layers "F.Cu" "B.Cu") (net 1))
 (via (at 199.5 28.5) (size 0.6) (drill 0.3) (layers "F.Cu" "B.Cu") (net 1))
 (via (at 206.04 33) (size 0.6) (drill 0.3) (layers "F.Cu" "B.Cu") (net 1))
 (segment (start 200.45 28.5) (end 200.95 28) (width 0.2) (layer "B.Cu") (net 1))
 (segment (start 204.289 34.5) (end 204.54 34.5) (width 0.2) (layer "B.Cu") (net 1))
 (segment (start 201.5 33.5) (end 201.5 33.1) (width 0.2) (layer "B.Cu") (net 1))
 (segment (start 204.54 34.5) (end 206.04 33) (width 0.2) (layer "B.Cu") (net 1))
 (segment (start 217.95 47.9) (end 217.95 41.95) (width 0.2) (layer "B.Cu") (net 1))
 (segment (start 217.95 41.95) (end 217.5 41.5) (width 0.2) (layer "B.Cu") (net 1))
 (segment (start 201.5 33.1) (end 204.1 30.5) (width 0.2) (layer "B.Cu") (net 1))
 (segment (start 199.5 28.5) (end 200.45 28.5) (width 0.2) (layer "B.Cu") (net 1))
 (segment (start 200.95 28) (end 199 29.95) (width 0.2) (layer "B.Cu") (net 1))
 (segment (start 199 29.95) (end 199 33) (width 0.2) (layer "B.Cu") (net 1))
 (segment (start 208.499 51.901) (end 203.16 57.24) (width 0.2) (layer "B.Cu") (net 6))
 (segment (start 217.95 51.1) (end 217.149 51.901) (width 0.2) (layer "B.Cu") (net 6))
 (segment (start 217.149 51.901) (end 208.499 51.901) (width 0.2) (layer "B.Cu") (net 6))
 (segment (start 216.45 25) (end 215.5 25) (width 0.2) (layer "F.Cu") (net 15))
 (segment (start 217.74 23.71) (end 216.45 25) (width 0.2) (layer "F.Cu") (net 15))
 (segment (start 207.5 38) (end 207 37.5) (width 0.2) (layer "F.Cu") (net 15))
 (segment (start 207 37.5) (end 206 37.5) (width 0.2) (layer "F.Cu") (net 15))
 (segment (start 207.5 38.5) (end 207.5 38) (width 0.2) (layer "F.Cu") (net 15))
 (via (at 206 37.5) (size 0.6) (drill 0.3) (layers "F.Cu" "B.Cu") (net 15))
 (via (at 215.5 25) (size 0.6) (drill 0.3) (layers "F.Cu" "B.Cu") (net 15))
 (via (at 207.5 38.5) (size 0.6) (drill 0.3) (layers "F.Cu" "B.Cu") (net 15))
 (segment (start 203.5 28) (end 207.449943 28) (width 0.2) (layer "B.Cu") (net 15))
 (segment (start 203.5 28) (end 212.5 28) (width 0.2) (layer "B.Cu") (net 15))
 (segment (start 206 35.59) (end 206.04 35.55) (width 0.2) (layer "B.Cu") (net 15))
 (segment (start 208.201 28.751057) (end 208.201 37.799) (width 0.2) (layer "B.Cu") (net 15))
 (segment (start 206 37.5) (end 206 35.59) (width 0.2) (layer "B.Cu") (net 15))
 (segment (start 212.5 28) (end 215.5 25) (width 0.2) (layer "B.Cu") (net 15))
 (segment (start 207.449943 28) (end 208.201 28.751057) (width 0.2) (layer "B.Cu") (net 15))
 (segment (start 208.201 37.799) (end 207.5 38.5) (width 0.2) (layer "B.Cu") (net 15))
 (segment (start 205.439 32.261) (end 205.439 33.989) (width 0.2) (layer "F.Cu") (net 16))
 (segment (start 205.439 33.989) (end 215.5 44.05) (width 0.2) (layer "F.Cu") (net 16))
 (segment (start 205.439 32.261) (end 206.189 32.261) (width 0.2) (layer "F.Cu") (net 16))
 (segment (start 206.189 32.261) (end 214.74 23.71) (width 0.2) (layer "F.Cu") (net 16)))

